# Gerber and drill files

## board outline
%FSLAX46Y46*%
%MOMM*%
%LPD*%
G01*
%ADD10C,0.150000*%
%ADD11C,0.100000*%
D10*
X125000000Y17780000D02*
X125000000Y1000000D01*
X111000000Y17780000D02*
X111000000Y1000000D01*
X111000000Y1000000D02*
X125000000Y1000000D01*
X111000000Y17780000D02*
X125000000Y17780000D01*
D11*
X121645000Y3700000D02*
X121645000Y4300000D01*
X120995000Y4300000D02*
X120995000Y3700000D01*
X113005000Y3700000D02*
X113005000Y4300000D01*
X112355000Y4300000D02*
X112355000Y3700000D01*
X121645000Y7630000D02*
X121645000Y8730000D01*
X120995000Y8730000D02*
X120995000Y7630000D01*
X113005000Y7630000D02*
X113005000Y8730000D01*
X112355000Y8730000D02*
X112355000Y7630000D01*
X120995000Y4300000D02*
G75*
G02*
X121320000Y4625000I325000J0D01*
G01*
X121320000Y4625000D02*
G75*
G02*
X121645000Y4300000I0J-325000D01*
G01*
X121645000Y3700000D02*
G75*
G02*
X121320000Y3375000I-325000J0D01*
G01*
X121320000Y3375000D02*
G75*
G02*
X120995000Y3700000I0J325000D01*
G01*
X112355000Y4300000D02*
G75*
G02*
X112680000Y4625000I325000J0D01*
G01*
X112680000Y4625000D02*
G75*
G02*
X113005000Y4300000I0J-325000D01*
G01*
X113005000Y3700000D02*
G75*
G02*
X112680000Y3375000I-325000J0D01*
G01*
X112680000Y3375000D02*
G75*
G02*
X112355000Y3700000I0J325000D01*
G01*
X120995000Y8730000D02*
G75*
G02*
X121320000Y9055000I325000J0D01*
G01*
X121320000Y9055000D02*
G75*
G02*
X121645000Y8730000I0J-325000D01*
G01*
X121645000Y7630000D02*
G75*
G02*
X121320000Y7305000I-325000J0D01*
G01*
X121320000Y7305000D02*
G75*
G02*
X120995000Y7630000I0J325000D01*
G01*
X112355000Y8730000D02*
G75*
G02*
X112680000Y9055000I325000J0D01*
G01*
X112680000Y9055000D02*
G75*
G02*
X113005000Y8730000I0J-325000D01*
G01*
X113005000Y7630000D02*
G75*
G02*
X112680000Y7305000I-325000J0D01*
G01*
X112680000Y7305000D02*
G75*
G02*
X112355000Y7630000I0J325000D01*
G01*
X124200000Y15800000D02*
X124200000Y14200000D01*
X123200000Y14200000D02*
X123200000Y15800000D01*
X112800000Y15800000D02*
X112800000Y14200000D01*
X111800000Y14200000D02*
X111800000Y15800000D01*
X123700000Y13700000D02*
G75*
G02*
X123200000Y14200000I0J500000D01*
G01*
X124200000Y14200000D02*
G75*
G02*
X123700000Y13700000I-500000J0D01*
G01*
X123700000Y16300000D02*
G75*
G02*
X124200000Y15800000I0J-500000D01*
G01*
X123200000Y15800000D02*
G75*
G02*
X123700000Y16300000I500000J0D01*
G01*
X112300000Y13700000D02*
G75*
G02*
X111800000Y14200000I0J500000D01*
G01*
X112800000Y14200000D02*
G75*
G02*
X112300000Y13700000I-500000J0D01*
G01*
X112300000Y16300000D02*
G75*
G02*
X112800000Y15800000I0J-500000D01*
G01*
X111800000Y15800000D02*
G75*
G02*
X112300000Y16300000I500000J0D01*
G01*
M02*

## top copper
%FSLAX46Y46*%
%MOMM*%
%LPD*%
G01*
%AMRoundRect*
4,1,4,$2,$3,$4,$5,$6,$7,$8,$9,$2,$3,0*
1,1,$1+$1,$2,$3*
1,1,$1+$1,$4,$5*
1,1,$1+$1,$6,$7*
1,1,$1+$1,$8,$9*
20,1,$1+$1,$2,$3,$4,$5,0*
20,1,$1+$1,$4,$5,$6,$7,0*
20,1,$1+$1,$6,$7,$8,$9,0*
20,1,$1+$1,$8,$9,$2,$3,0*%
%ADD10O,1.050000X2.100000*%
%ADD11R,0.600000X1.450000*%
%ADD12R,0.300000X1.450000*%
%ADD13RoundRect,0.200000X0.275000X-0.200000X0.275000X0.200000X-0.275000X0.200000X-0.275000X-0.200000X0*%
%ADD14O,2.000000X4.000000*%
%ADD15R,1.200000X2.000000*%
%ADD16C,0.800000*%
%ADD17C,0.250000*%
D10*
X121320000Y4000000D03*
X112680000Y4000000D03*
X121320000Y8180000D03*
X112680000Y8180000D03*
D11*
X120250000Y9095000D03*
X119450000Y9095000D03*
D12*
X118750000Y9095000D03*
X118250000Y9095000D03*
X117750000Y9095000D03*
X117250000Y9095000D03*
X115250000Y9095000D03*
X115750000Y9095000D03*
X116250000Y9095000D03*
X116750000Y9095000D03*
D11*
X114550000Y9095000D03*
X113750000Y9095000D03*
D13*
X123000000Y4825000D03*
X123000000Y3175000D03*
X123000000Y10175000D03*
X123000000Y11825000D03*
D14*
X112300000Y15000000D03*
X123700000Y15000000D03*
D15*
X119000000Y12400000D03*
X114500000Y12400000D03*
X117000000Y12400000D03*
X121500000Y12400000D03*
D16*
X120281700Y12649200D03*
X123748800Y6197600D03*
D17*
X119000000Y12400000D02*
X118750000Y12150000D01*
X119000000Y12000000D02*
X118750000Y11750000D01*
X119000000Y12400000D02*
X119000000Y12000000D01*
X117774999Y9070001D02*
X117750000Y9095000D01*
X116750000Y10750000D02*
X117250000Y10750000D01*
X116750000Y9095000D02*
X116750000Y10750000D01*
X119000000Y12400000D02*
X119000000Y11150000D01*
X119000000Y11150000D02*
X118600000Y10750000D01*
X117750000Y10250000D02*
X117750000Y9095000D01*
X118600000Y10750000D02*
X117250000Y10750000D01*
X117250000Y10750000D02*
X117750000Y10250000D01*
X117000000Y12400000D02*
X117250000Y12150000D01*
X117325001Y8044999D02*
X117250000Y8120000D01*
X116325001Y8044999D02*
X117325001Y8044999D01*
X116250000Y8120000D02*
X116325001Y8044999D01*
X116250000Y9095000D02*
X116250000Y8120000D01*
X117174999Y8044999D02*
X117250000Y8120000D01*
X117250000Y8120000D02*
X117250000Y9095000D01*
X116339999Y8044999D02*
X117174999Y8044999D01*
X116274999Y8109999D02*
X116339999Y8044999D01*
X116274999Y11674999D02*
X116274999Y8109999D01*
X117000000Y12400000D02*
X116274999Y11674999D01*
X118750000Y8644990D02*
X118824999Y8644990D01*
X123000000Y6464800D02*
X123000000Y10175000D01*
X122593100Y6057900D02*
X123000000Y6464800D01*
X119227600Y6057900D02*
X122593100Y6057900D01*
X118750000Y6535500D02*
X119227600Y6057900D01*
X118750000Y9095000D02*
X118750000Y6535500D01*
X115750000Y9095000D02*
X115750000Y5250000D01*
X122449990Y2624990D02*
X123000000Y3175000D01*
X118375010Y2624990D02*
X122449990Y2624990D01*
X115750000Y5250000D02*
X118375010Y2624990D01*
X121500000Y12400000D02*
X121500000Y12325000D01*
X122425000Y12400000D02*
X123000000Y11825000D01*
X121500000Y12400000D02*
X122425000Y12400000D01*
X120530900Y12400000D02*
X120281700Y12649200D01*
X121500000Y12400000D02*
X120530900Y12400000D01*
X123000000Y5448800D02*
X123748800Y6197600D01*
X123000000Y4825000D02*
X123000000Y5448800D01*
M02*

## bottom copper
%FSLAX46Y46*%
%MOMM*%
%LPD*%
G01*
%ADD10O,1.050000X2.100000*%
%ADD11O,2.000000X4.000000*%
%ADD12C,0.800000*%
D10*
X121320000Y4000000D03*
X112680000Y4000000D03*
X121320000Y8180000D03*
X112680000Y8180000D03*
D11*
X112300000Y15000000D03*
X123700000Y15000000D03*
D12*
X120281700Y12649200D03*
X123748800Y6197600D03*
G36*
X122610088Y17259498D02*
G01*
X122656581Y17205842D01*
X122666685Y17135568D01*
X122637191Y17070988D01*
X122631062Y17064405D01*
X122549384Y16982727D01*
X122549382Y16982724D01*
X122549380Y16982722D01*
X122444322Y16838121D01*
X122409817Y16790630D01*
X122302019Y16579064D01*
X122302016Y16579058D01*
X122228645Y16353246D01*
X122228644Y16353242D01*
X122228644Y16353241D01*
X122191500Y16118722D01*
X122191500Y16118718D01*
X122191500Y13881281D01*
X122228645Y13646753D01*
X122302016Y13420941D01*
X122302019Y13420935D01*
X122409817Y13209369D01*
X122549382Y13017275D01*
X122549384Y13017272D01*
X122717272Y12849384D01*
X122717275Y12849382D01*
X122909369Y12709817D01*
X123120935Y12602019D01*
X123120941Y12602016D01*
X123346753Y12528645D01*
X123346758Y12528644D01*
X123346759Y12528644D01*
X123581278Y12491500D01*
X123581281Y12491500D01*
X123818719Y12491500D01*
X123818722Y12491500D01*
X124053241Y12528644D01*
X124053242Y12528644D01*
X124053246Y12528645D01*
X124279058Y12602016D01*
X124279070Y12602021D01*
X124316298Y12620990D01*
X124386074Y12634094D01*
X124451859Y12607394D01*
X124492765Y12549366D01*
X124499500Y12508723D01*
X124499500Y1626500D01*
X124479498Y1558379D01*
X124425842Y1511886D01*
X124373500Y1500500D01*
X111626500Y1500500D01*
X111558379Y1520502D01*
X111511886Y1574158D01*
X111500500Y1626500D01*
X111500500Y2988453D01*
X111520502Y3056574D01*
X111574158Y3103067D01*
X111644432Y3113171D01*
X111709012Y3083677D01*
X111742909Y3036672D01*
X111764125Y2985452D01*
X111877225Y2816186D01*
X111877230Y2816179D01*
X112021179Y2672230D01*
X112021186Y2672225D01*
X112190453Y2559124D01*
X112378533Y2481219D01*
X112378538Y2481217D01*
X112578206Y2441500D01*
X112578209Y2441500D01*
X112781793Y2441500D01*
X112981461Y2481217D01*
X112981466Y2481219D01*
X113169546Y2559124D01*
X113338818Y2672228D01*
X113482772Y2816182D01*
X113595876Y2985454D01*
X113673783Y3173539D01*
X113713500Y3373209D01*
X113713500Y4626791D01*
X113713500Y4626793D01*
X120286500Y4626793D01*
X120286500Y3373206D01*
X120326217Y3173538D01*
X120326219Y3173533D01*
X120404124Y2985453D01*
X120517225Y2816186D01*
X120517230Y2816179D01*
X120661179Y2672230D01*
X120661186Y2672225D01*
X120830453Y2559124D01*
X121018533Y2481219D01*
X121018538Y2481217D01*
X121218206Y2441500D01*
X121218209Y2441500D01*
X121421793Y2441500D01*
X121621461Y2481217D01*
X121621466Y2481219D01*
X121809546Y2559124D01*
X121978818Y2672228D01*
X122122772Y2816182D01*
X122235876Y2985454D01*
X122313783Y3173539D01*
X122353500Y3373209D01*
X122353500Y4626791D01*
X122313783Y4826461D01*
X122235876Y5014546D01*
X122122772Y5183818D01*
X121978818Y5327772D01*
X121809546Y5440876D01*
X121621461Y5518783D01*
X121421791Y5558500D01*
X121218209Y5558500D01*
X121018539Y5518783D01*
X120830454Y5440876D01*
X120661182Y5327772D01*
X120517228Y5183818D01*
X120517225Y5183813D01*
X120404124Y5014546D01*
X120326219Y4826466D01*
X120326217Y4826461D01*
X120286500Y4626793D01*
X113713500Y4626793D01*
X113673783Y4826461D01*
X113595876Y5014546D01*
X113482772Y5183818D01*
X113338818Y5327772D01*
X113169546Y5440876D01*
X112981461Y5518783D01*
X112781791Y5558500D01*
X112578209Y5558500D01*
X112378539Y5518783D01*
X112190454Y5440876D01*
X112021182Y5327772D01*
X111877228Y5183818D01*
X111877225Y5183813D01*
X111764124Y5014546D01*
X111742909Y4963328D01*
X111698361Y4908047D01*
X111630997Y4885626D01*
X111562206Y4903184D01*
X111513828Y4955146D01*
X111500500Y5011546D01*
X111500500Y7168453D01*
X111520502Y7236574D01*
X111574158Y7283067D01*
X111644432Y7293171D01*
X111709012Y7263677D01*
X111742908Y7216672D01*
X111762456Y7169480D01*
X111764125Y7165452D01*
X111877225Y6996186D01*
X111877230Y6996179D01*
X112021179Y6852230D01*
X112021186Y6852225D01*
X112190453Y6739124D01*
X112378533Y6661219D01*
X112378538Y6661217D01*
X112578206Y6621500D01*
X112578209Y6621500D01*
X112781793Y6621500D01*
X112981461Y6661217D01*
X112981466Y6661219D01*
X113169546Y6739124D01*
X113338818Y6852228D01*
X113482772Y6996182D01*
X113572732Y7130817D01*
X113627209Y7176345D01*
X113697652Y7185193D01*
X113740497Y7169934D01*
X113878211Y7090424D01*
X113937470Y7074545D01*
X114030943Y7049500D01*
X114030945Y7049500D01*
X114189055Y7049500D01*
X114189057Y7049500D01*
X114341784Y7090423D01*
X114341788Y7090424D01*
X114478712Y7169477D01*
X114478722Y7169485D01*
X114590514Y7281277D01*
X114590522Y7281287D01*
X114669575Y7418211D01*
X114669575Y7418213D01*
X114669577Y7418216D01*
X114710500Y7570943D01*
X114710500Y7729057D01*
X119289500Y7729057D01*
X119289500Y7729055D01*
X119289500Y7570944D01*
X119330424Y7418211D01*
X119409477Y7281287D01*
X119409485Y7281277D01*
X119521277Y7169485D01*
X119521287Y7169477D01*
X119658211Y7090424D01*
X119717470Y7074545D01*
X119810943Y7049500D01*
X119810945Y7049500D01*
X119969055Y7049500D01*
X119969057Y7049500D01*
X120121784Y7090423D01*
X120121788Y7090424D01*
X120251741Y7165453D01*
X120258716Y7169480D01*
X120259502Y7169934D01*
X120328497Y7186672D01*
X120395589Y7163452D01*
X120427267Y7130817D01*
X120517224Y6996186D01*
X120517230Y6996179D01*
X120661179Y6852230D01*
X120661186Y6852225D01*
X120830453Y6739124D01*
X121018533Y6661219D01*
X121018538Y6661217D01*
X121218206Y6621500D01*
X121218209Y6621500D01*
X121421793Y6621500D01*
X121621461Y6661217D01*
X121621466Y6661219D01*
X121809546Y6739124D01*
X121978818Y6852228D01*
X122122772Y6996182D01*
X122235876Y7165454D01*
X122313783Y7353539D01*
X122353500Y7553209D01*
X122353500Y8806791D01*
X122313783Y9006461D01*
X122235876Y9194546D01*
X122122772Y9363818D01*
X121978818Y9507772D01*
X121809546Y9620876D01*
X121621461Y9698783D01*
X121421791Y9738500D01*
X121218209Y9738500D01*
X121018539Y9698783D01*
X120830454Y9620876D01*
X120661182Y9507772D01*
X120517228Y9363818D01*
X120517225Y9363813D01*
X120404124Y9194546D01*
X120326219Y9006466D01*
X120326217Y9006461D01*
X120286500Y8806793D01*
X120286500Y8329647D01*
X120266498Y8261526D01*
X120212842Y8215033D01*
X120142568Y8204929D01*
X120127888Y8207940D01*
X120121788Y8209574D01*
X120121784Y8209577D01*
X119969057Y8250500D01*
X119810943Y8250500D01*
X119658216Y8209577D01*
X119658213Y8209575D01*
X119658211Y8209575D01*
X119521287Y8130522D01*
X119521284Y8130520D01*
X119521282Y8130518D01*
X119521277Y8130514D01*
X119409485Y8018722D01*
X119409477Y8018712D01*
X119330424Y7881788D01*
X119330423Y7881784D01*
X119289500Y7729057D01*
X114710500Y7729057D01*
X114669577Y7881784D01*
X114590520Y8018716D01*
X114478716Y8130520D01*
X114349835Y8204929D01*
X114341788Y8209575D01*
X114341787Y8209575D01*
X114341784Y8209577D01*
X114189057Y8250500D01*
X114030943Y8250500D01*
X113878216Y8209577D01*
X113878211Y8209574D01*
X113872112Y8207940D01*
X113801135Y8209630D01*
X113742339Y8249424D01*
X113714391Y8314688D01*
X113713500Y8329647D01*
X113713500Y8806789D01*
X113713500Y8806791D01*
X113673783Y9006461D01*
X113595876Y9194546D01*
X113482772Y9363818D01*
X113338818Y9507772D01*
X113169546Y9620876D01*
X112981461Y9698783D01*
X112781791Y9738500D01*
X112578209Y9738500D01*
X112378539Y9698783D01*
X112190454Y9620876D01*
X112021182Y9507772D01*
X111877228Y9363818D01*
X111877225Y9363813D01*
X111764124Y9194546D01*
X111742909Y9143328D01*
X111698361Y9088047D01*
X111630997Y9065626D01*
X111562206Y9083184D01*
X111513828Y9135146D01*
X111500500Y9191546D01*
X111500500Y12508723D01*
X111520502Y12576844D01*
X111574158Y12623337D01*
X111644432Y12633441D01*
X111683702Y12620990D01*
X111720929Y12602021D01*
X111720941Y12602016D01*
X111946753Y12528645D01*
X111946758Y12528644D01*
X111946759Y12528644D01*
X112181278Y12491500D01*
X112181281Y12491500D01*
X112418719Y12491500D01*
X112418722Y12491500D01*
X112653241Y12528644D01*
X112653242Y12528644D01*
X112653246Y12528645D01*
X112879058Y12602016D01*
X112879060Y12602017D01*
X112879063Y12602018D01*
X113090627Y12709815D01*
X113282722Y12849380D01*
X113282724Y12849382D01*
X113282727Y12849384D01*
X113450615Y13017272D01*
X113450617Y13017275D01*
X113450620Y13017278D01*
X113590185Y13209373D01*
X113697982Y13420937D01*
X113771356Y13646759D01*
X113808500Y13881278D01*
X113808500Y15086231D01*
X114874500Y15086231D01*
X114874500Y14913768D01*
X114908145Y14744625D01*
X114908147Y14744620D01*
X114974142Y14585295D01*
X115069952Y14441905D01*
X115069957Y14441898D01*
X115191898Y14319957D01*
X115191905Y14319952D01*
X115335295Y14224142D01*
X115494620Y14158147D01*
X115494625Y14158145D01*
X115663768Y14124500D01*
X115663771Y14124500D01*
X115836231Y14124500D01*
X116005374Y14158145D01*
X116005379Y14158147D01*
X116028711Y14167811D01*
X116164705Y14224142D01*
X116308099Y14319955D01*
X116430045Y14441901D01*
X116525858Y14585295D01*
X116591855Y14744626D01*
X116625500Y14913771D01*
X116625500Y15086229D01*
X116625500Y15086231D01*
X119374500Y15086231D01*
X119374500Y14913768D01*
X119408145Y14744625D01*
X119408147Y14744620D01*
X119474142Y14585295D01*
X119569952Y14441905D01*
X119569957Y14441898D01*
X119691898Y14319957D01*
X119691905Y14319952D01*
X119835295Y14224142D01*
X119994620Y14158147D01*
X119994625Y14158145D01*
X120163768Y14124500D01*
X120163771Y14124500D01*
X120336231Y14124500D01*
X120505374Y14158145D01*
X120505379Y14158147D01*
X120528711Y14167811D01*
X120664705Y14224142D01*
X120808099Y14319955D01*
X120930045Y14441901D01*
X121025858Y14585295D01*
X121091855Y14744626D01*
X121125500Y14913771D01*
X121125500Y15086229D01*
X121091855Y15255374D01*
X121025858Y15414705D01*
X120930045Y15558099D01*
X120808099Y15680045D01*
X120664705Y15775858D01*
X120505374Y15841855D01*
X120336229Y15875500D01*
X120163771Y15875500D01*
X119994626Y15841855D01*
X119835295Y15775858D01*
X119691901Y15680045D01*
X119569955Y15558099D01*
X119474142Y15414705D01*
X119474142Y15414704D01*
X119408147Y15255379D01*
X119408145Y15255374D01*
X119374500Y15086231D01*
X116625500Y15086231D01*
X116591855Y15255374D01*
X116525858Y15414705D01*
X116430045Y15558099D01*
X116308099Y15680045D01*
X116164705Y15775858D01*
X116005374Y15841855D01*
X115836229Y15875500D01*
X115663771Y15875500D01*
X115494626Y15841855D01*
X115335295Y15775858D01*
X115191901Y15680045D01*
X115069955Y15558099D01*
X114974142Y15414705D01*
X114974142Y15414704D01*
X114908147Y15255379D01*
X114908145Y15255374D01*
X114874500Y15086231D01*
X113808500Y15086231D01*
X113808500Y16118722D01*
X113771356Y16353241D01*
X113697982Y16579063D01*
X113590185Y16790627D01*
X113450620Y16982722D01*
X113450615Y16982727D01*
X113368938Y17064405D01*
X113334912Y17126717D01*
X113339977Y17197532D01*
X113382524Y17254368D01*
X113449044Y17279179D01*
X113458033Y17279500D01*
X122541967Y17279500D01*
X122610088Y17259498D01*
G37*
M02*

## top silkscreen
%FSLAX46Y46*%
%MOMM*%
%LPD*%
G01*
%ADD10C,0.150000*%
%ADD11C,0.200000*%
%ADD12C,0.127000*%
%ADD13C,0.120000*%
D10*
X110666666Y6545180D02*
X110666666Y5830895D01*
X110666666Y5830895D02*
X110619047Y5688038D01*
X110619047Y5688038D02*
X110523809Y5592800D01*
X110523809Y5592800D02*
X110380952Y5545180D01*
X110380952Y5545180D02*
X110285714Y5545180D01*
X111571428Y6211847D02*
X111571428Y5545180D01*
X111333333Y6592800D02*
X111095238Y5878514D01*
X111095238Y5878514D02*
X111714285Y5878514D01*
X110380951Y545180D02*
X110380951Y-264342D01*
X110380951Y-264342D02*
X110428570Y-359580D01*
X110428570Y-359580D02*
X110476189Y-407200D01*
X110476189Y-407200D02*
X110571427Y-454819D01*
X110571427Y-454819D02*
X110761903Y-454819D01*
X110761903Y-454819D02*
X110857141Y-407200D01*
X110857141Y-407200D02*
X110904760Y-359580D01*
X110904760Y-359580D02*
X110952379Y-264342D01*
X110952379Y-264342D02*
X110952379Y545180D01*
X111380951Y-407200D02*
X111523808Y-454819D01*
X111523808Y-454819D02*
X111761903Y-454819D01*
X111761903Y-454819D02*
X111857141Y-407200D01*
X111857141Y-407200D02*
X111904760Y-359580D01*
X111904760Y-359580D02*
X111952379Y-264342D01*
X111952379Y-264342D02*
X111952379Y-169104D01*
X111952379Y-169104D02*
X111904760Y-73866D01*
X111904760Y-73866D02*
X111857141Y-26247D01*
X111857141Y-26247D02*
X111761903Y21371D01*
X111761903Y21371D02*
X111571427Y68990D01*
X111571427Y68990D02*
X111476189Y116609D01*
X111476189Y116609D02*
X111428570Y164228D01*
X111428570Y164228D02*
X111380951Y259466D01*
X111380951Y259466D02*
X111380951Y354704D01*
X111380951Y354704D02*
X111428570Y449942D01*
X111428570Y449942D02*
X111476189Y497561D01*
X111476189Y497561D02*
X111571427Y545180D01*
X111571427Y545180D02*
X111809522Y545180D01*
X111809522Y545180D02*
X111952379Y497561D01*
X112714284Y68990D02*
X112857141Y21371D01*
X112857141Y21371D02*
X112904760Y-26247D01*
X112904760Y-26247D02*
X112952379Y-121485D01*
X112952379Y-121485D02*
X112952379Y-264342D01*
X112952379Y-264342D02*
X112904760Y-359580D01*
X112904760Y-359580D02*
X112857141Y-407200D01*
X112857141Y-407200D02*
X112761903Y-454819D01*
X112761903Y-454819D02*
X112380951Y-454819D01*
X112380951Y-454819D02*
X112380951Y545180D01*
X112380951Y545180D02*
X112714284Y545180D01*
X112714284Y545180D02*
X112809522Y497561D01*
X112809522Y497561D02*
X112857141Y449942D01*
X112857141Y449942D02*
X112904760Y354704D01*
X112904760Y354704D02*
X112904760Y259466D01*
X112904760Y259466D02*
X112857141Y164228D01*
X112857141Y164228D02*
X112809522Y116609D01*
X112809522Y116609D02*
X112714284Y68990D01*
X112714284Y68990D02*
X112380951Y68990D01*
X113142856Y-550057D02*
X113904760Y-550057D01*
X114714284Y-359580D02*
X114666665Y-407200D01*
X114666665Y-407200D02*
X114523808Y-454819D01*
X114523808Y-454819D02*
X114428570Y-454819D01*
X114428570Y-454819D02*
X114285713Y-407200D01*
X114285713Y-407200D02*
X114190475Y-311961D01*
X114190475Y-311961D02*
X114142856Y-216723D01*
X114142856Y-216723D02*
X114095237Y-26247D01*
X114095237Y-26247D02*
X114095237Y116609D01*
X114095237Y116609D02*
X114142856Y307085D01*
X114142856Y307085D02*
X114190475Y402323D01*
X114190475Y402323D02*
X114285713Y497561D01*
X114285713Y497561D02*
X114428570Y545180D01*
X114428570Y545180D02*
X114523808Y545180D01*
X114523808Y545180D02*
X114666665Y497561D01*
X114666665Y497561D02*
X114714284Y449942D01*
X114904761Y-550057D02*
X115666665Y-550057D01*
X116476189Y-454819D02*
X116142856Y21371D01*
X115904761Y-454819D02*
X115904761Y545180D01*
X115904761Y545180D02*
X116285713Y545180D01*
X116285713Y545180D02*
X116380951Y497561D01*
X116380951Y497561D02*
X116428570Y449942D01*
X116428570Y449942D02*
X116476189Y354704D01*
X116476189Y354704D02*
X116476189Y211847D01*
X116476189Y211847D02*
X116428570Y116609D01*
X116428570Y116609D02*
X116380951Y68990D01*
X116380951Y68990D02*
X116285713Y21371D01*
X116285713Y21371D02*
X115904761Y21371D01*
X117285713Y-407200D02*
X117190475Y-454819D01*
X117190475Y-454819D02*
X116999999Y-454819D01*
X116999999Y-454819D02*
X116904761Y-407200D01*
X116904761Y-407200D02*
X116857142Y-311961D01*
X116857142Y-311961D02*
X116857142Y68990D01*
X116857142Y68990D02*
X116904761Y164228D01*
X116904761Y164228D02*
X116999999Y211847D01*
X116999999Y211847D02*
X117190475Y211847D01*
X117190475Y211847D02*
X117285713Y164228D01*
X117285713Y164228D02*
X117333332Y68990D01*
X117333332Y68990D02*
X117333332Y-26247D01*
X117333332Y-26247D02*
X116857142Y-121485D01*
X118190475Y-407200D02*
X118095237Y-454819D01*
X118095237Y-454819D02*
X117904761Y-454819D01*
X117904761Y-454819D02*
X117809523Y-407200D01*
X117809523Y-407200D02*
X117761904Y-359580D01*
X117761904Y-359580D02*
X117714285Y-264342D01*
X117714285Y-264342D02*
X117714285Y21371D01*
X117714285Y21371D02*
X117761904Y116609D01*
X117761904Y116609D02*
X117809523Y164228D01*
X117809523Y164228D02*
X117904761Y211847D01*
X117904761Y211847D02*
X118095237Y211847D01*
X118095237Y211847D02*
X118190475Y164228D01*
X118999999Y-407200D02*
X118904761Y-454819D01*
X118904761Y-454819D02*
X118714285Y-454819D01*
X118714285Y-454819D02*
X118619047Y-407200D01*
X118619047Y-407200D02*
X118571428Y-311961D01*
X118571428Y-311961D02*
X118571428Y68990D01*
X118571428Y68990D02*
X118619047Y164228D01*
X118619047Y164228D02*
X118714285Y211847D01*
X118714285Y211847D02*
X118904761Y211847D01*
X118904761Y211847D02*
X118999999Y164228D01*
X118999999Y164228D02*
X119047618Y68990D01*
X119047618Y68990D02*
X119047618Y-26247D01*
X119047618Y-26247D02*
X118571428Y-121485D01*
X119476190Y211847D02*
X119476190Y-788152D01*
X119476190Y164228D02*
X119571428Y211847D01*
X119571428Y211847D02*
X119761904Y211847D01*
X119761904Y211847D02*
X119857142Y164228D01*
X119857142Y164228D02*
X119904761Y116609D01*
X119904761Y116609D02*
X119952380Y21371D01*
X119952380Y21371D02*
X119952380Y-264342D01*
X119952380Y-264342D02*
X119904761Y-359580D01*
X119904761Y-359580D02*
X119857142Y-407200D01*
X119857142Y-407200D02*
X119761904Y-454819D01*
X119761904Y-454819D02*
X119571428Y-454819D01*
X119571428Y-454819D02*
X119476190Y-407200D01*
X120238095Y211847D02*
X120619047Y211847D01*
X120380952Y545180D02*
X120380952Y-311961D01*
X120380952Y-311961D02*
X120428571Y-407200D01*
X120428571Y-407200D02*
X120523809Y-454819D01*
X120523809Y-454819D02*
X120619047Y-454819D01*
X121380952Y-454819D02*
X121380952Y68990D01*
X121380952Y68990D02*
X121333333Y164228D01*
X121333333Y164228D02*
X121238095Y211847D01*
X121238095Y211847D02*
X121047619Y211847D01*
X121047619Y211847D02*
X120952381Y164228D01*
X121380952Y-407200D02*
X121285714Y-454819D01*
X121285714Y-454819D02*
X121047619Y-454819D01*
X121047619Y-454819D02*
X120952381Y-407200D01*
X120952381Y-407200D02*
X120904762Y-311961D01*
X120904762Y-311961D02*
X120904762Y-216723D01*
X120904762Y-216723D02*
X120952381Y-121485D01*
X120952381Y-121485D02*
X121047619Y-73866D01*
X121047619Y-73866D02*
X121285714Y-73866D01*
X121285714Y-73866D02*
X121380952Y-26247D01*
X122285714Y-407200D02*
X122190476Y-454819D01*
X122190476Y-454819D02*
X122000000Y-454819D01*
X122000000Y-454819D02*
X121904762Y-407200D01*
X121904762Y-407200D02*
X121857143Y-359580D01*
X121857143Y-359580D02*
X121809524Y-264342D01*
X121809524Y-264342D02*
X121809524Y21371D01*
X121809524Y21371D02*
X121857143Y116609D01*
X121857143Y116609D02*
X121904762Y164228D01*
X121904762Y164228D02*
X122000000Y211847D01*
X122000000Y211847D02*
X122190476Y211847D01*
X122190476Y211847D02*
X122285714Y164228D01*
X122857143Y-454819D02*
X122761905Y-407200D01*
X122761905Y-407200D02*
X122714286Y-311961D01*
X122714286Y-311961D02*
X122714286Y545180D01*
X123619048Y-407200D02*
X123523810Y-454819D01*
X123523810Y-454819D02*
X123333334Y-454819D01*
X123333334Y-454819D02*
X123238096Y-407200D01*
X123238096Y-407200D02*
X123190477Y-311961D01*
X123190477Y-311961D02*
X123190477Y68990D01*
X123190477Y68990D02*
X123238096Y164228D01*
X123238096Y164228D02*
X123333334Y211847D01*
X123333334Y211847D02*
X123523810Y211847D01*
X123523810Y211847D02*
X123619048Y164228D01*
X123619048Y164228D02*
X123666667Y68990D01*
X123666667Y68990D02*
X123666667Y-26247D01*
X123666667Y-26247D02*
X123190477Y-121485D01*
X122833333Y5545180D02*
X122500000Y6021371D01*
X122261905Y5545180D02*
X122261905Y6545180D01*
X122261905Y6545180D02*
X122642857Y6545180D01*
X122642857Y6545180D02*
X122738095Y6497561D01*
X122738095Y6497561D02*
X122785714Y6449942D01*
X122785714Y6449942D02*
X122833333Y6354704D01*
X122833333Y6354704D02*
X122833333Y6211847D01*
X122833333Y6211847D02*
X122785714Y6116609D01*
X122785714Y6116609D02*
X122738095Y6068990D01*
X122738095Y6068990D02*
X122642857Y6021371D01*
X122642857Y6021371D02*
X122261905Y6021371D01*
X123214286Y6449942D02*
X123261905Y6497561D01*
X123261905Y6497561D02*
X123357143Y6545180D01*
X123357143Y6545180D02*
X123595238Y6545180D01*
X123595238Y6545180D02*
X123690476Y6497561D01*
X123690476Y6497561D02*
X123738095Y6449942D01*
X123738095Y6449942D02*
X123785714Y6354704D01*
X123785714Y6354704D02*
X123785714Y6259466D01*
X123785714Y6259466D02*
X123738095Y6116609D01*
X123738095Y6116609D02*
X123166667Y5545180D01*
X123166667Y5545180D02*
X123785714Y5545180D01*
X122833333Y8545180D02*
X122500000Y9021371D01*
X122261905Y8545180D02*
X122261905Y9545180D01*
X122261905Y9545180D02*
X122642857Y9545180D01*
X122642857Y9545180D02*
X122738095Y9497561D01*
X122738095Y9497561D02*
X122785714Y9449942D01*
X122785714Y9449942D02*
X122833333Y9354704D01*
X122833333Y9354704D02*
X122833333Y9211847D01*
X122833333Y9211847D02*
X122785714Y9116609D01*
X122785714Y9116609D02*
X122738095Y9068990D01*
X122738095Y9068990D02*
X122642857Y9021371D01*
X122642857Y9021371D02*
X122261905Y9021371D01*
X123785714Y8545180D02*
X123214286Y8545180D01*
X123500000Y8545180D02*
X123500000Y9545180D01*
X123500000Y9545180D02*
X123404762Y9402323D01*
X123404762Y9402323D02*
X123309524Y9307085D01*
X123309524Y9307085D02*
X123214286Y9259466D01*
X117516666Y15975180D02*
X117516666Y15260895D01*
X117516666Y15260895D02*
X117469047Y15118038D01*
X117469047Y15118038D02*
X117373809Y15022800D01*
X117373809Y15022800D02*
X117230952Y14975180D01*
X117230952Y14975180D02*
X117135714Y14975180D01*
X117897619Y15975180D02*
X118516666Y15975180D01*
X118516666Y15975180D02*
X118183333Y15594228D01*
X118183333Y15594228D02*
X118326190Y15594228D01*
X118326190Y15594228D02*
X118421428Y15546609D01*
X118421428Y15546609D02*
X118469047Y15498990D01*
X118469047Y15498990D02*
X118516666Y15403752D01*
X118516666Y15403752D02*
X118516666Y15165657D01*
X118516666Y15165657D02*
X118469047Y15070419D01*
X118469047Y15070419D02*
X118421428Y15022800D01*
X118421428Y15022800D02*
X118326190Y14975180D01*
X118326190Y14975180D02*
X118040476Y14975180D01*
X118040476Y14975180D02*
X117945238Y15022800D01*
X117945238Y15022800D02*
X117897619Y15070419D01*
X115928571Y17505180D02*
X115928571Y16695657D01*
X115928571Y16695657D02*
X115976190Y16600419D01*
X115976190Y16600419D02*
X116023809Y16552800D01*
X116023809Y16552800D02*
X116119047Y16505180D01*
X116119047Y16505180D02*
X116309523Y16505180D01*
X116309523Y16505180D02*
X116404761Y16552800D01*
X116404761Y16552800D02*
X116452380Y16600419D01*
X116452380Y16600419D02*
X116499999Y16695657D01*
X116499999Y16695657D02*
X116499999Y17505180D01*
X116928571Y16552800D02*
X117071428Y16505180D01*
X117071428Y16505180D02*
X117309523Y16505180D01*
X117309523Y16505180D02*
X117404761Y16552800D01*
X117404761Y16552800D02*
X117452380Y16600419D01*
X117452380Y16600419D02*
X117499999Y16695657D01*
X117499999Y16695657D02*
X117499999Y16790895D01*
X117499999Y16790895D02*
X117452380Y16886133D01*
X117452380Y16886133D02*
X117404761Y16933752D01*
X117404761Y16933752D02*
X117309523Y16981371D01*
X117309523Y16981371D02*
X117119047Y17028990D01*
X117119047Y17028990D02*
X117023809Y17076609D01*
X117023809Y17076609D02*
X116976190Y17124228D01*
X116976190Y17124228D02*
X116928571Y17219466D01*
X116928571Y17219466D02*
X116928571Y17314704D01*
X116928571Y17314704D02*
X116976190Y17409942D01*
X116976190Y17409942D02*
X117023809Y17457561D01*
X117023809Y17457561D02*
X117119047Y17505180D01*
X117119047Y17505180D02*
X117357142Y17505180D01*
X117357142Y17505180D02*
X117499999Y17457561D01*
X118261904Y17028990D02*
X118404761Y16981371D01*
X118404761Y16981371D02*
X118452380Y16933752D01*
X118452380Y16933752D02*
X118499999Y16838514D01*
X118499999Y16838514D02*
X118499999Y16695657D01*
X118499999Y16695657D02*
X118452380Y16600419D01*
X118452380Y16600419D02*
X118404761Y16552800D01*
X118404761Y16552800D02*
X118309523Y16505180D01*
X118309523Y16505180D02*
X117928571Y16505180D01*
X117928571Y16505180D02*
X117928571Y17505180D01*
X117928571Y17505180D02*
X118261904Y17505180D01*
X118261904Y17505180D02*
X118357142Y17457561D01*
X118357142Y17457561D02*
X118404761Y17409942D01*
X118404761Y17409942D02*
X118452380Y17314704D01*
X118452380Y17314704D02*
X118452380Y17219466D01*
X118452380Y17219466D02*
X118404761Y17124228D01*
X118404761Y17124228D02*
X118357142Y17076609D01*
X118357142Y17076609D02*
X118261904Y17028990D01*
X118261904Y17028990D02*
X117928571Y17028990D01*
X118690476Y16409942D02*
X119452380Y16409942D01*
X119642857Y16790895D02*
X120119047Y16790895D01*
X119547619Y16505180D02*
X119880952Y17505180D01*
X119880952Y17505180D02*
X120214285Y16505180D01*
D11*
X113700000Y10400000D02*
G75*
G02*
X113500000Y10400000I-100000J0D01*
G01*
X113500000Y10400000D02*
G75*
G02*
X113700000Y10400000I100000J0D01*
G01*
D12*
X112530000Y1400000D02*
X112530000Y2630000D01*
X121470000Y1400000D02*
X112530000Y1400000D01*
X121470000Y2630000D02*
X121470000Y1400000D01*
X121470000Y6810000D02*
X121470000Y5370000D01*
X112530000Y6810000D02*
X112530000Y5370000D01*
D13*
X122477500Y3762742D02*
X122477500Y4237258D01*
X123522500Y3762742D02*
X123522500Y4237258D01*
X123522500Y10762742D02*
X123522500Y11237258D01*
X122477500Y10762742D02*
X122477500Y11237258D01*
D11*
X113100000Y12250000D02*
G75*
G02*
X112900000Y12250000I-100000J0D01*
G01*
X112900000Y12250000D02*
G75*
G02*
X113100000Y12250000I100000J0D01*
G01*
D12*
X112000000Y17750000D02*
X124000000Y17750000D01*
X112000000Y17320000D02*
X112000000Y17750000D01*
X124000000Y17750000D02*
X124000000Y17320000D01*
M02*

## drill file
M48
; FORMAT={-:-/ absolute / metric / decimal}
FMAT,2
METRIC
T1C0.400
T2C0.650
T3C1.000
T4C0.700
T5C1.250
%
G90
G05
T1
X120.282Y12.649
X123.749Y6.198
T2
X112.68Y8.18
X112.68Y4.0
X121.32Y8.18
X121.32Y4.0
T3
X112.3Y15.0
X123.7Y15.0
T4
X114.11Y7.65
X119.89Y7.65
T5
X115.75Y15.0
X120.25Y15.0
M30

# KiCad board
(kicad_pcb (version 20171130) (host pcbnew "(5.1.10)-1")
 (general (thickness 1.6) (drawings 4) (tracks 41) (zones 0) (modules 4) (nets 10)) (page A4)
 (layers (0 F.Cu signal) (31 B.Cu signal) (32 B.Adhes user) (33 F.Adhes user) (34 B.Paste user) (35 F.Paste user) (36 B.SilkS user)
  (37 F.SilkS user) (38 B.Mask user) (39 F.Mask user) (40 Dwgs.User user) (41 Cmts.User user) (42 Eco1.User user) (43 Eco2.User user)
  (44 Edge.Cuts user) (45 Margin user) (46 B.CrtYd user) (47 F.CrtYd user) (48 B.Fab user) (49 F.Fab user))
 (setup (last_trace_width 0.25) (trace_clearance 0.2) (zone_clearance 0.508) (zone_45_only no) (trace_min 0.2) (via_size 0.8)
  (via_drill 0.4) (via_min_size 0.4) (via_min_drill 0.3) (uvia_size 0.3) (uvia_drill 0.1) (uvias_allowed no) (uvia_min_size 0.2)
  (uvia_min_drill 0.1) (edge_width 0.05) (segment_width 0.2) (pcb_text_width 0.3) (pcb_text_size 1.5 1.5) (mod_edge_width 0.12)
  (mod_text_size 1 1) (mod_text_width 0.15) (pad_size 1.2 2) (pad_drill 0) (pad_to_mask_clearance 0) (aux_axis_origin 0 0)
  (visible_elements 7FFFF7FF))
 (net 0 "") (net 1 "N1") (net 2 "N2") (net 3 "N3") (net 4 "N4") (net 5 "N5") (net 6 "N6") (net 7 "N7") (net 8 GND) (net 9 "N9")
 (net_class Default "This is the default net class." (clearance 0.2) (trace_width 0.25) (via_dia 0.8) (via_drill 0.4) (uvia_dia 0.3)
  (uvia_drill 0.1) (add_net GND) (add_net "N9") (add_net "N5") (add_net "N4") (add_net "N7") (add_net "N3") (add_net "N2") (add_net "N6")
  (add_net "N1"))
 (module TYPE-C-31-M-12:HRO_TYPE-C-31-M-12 (layer F.Cu) (at 117 -4)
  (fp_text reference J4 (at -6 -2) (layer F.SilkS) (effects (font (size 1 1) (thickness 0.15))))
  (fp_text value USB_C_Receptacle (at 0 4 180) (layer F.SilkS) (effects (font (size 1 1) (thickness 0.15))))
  (fp_circle (center -3.4 -6.4) (end -3.3 -6.4) (layer F.SilkS) (width 0.2))
  (fp_line (start -4.47 2.6) (end -4.47 1.37) (layer F.SilkS) (width 0.127))
  (fp_line (start 4.47 2.6) (end -4.47 2.6) (layer F.SilkS) (width 0.127))
  (fp_line (start 4.47 1.37) (end 4.47 2.6) (layer F.SilkS) (width 0.127))
  (fp_line (start 4.47 -2.81) (end 4.47 -1.37) (layer F.SilkS) (width 0.127))
  (fp_line (start -4.47 -2.81) (end -4.47 -1.37) (layer F.SilkS) (width 0.127))
  (fp_line (start 4.645 0.3) (end 4.645 -0.3) (layer Edge.Cuts) (width 0.1))
  (fp_line (start 3.995 -0.3) (end 3.995 0.3) (layer Edge.Cuts) (width 0.1))
  (fp_line (start -3.995 0.3) (end -3.995 -0.3) (layer Edge.Cuts) (width 0.1))
  (fp_line (start -4.645 -0.3) (end -4.645 0.3) (layer Edge.Cuts) (width 0.1))
  (fp_line (start 4.645 -3.63) (end 4.645 -4.73) (layer Edge.Cuts) (width 0.1))
  (fp_line (start 3.995 -4.73) (end 3.995 -3.63) (layer Edge.Cuts) (width 0.1))
  (fp_line (start -3.995 -3.63) (end -3.995 -4.73) (layer Edge.Cuts) (width 0.1))
  (fp_line (start -4.645 -4.73) (end -4.645 -3.63) (layer Edge.Cuts) (width 0.1))
  (fp_arc (start 4.32 -0.3) (end 3.995 -0.3) (angle 90) (layer Edge.Cuts) (width 0.1))
  (fp_arc (start 4.32 -0.3) (end 4.32 -0.625) (angle 90) (layer Edge.Cuts) (width 0.1))
  (fp_arc (start 4.32 0.3) (end 4.645 0.3) (angle 90) (layer Edge.Cuts) (width 0.1))
  (fp_arc (start 4.32 0.3) (end 4.32 0.625) (angle 90) (layer Edge.Cuts) (width 0.1))
  (fp_arc (start -4.32 -0.3) (end -4.645 -0.3) (angle 90) (layer Edge.Cuts) (width 0.1))
  (fp_arc (start -4.32 -0.3) (end -4.32 -0.625) (angle 90) (layer Edge.Cuts) (width 0.1))
  (fp_arc (start -4.32 0.3) (end -3.995 0.3) (angle 90) (layer Edge.Cuts) (width 0.1))
  (fp_arc (start -4.32 0.3) (end -4.32 0.625) (angle 90) (layer Edge.Cuts) (width 0.1))
  (fp_arc (start 4.32 -4.73) (end 3.995 -4.73) (angle 90) (layer Edge.Cuts) (width 0.1))
  (fp_arc (start 4.32 -4.73) (end 4.32 -5.055) (angle 90) (layer Edge.Cuts) (width 0.1))
  (fp_arc (start 4.32 -3.63) (end 4.645 -3.63) (angle 90) (layer Edge.Cuts) (width 0.1))
  (fp_arc (start 4.32 -3.63) (end 4.32 -3.305) (angle 90) (layer Edge.Cuts) (width 0.1))
  (fp_arc (start -4.32 -4.73) (end -4.645 -4.73) (angle 90) (layer Edge.Cuts) (width 0.1))
  (fp_arc (start -4.32 -4.73) (end -4.32 -5.055) (angle 90) (layer Edge.Cuts) (width 0.1))
  (fp_arc (start -4.32 -3.63) (end -3.995 -3.63) (angle 90) (layer Edge.Cuts) (width 0.1))
  (fp_arc (start -4.32 -3.63) (end -4.32 -3.305) (angle 90) (layer Edge.Cuts) (width 0.1))
  (pad Hole np_thru_hole circle (at 2.89 -3.65) (size 0.7 0.7) (drill 0.7) (layers *.Cu *.Mask))
  (pad Hole np_thru_hole circle (at -2.89 -3.65) (size 0.7 0.7) (drill 0.7) (layers *.Cu *.Mask))
  (pad S4 thru_hole oval (at 4.32 0 90) (size 2.1 1.05) (drill 0.65) (layers *.Cu *.Mask))
  (pad S3 thru_hole oval (at -4.32 0 90) (size 2.1 1.05) (drill 0.65) (layers *.Cu *.Mask))
  (pad S2 thru_hole oval (at 4.32 -4.18 90) (size 2.1 1.05) (drill 0.65) (layers *.Cu *.Mask))
  (pad S1 thru_hole oval (at -4.32 -4.18 90) (size 2.1 1.05) (drill 0.65) (layers *.Cu *.Mask) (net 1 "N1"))
  (pad B1A12 smd rect (at 3.25 -5.095) (size 0.6 1.45) (layers F.Cu F.Paste))
  (pad B4A9 smd rect (at 2.45 -5.095) (size 0.6 1.45) (layers F.Cu F.Paste))
  (pad B5 smd rect (at 1.75 -5.095) (size 0.3 1.45) (layers F.Cu F.Paste) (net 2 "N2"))
  (pad A8 smd rect (at 1.25 -5.095) (size 0.3 1.45) (layers F.Cu F.Paste) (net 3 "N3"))
  (pad B6 smd rect (at 0.75 -5.095) (size 0.3 1.45) (layers F.Cu F.Paste) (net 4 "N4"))
  (pad A7 smd rect (at 0.25 -5.095) (size 0.3 1.45) (layers F.Cu F.Paste) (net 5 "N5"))
  (pad B8 smd rect (at -1.75 -5.095) (size 0.3 1.45) (layers F.Cu F.Paste) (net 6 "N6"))
  (pad A5 smd rect (at -1.25 -5.095) (size 0.3 1.45) (layers F.Cu F.Paste) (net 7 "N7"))
  (pad B7 smd rect (at -0.75 -5.095) (size 0.3 1.45) (layers F.Cu F.Paste) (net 5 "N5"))
  (pad A6 smd rect (at -0.25 -5.095) (size 0.3 1.45) (layers F.Cu F.Paste) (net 4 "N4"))
  (pad A4B9 smd rect (at -2.45 -5.095) (size 0.6 1.45) (layers F.Cu F.Paste))
  (pad A1B12 smd rect (at -3.25 -5.095) (size 0.6 1.45) (layers F.Cu F.Paste)))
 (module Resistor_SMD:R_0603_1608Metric (layer F.Cu) (at 123 -4 90)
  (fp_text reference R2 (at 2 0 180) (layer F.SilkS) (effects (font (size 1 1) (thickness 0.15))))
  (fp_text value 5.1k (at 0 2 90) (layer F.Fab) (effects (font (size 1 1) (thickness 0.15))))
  (fp_line (start -0.237258 -0.5225) (end 0.237258 -0.5225) (layer F.SilkS) (width 0.12))
  (fp_line (start -0.237258 0.5225) (end 0.237258 0.5225) (layer F.SilkS) (width 0.12))
  (pad 2 smd roundrect (at 0.825 0 90) (size 0.8 0.95) (layers F.Cu F.Paste F.Mask) (roundrect_rratio 0.25) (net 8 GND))
  (pad 1 smd roundrect (at -0.825 0 90) (size 0.8 0.95) (layers F.Cu F.Paste F.Mask) (roundrect_rratio 0.25) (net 7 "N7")))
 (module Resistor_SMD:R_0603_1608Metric (layer F.Cu) (at 123 -11 90)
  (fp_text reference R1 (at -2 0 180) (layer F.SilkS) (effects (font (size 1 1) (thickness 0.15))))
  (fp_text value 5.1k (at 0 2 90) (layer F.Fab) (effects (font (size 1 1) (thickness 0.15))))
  (fp_line (start -0.237258 0.5225) (end 0.237258 0.5225) (layer F.SilkS) (width 0.12))
  (fp_line (start -0.237258 -0.5225) (end 0.237258 -0.5225) (layer F.SilkS) (width 0.12))
  (pad 1 smd roundrect (at -0.825 0 90) (size 0.8 0.95) (layers F.Cu F.Paste F.Mask) (roundrect_rratio 0.25) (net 2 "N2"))
  (pad 2 smd roundrect (at 0.825 0 90) (size 0.8 0.95) (layers F.Cu F.Paste F.Mask) (roundrect_rratio 0.25) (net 8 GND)))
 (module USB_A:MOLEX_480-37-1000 (layer F.Cu) (at 118 -15 180)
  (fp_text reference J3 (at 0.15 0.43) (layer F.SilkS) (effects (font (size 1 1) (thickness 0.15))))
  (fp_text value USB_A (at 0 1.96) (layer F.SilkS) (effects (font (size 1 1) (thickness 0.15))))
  (fp_line (start -6.2 0.8) (end -6.2 -0.8) (layer Edge.Cuts) (width 0.1))
  (fp_line (start -5.2 -0.8) (end -5.2 0.8) (layer Edge.Cuts) (width 0.1))
  (fp_line (start 5.2 0.8) (end 5.2 -0.8) (layer Edge.Cuts) (width 0.1))
  (fp_line (start 6.2 -0.8) (end 6.2 0.8) (layer Edge.Cuts) (width 0.1))
  (fp_circle (center 5 -2.75) (end 5.1 -2.75) (layer F.SilkS) (width 0.2))
  (fp_line (start 6 2.75) (end -6 2.75) (layer F.SilkS) (width 0.127))
  (fp_line (start 6 2.32) (end 6 2.75) (layer F.SilkS) (width 0.127))
  (fp_line (start -6 2.75) (end -6 2.32) (layer F.SilkS) (width 0.127))
  (fp_arc (start -5.7 -0.8) (end -5.2 -0.8) (angle -90) (layer Edge.Cuts) (width 0.1))
  (fp_arc (start -5.7 -0.8) (end -5.7 -1.3) (angle -90) (layer Edge.Cuts) (width 0.1))
  (fp_arc (start -5.7 0.8) (end -6.2 0.8) (angle -90) (layer Edge.Cuts) (width 0.1))
  (fp_arc (start -5.7 0.8) (end -5.7 1.3) (angle -90) (layer Edge.Cuts) (width 0.1))
  (fp_arc (start 5.7 -0.8) (end 6.2 -0.8) (angle -90) (layer Edge.Cuts) (width 0.1))
  (fp_arc (start 5.7 -0.8) (end 5.7 -1.3) (angle -90) (layer Edge.Cuts) (width 0.1))
  (fp_arc (start 5.7 0.8) (end 5.2 0.8) (angle -90) (layer Edge.Cuts) (width 0.1))
  (fp_arc (start 5.7 0.8) (end 5.7 1.3) (angle -90) (layer Edge.Cuts) (width 0.1))
  (pad S2 thru_hole oval (at 5.7 0 270) (size 4 2) (drill 1) (layers *.Cu *.Mask))
  (pad S1 thru_hole oval (at -5.7 0 270) (size 4 2) (drill 1) (layers *.Cu *.Mask))
  (pad 3 smd rect (at -1 -2.6 180) (size 1.2 2) (layers F.Cu F.Paste) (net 4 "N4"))
  (pad 1 smd rect (at 3.5 -2.6 180) (size 1.2 2) (layers F.Cu F.Paste) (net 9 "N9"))
  (pad 2 smd rect (at 1 -2.6 180) (size 1.2 2) (layers F.Cu F.Paste) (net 5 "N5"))
  (pad 4 smd rect (at -3.5 -2.6 180) (size 1.2 2) (layers F.Cu F.Paste) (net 8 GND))
  (pad Hole np_thru_hole circle (at 2.25 0 180) (size 1.25 1.25) (drill 1.25) (layers *.Cu *.Mask))
  (pad Hole np_thru_hole circle (at -2.25 0 180) (size 1.25 1.25) (drill 1.25) (layers *.Cu *.Mask)))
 (gr_line (start 125 -17.78) (end 125 -1) (layer Edge.Cuts) (width 0.15))
 (gr_line (start 111 -17.78) (end 111 -1) (layer Edge.Cuts) (width 0.15))
 (gr_line (start 111 -1) (end 125 -1) (layer Edge.Cuts) (width 0.15))
 (gr_line (start 111 -17.78) (end 125 -17.78) (layer Edge.Cuts) (width 0.15))
 (segment (start 119 -12.4) (end 118.75 -12.15) (width 0.25) (layer F.Cu) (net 4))
 (segment (start 119 -12) (end 118.75 -11.75) (width 0.25) (layer F.Cu) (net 4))
 (segment (start 119 -12.4) (end 119 -12) (width 0.25) (layer F.Cu) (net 4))
 (segment (start 117.774999 -9.070001) (end 117.75 -9.095) (width 0.25) (layer F.Cu) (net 4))
 (segment (start 116.75 -10.75) (end 117.25 -10.75) (width 0.25) (layer F.Cu) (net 4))
 (segment (start 116.75 -9.095) (end 116.75 -10.75) (width 0.25) (layer F.Cu) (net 4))
 (segment (start 119 -12.4) (end 119 -11.15) (width 0.25) (layer F.Cu) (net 4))
 (segment (start 119 -11.15) (end 118.6 -10.75) (width 0.25) (layer F.Cu) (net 4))
 (segment (start 117.75 -10.25) (end 117.75 -9.095) (width 0.25) (layer F.Cu) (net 4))
 (segment (start 118.6 -10.75) (end 117.25 -10.75) (width 0.25) (layer F.Cu) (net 4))
 (segment (start 117.25 -10.75) (end 117.75 -10.25) (width 0.25) (layer F.Cu) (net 4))
 (segment (start 117 -12.4) (end 117.25 -12.15) (width 0.25) (layer F.Cu) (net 5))
 (segment (start 117.325001 -8.044999) (end 117.25 -8.12) (width 0.25) (layer F.Cu) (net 5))
 (segment (start 116.325001 -8.044999) (end 117.325001 -8.044999) (width 0.25) (layer F.Cu) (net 5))
 (segment (start 116.25 -8.12) (end 116.325001 -8.044999) (width 0.25) (layer F.Cu) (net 5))
 (segment (start 116.25 -9.095) (end 116.25 -8.12) (width 0.25) (layer F.Cu) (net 5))
 (segment (start 117.174999 -8.044999) (end 117.25 -8.12) (width 0.25) (layer F.Cu) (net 5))
 (segment (start 117.25 -8.12) (end 117.25 -9.095) (width 0.25) (layer F.Cu) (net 5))
 (segment (start 116.339999 -8.044999) (end 117.174999 -8.044999) (width 0.25) (layer F.Cu) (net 5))
 (segment (start 116.274999 -8.109999) (end 116.339999 -8.044999) (width 0.25) (layer F.Cu) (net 5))
 (segment (start 116.274999 -11.674999) (end 116.274999 -8.109999) (width 0.25) (layer F.Cu) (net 5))
 (segment (start 117 -12.4) (end 116.274999 -11.674999) (width 0.25) (layer F.Cu) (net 5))
 (segment (start 118.75 -8.64499) (end 118.824999 -8.64499) (width 0.25) (layer F.Cu) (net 2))
 (segment (start 123 -6.4648) (end 123 -10.175) (width 0.25) (layer F.Cu) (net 2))
 (segment (start 122.5931 -6.0579) (end 123 -6.4648) (width 0.25) (layer F.Cu) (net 2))
 (segment (start 119.2276 -6.0579) (end 122.5931 -6.0579) (width 0.25) (layer F.Cu) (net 2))
 (segment (start 118.75 -6.5355) (end 119.2276 -6.0579) (width 0.25) (layer F.Cu) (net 2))
 (segment (start 118.75 -9.095) (end 118.75 -6.5355) (width 0.25) (layer F.Cu) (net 2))
 (segment (start 115.75 -9.095) (end 115.75 -5.25) (width 0.25) (layer F.Cu) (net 7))
 (segment (start 122.44999 -2.62499) (end 123 -3.175) (width 0.25) (layer F.Cu) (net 7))
 (segment (start 118.37501 -2.62499) (end 122.44999 -2.62499) (width 0.25) (layer F.Cu) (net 7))
 (segment (start 115.75 -5.25) (end 118.37501 -2.62499) (width 0.25) (layer F.Cu) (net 7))
 (segment (start 121.5 -12.4) (end 121.5 -12.325) (width 0.25) (layer F.Cu) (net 8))
 (segment (start 122.425 -12.4) (end 123 -11.825) (width 0.25) (layer F.Cu) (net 8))
 (segment (start 121.5 -12.4) (end 122.425 -12.4) (width 0.25) (layer F.Cu) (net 8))
 (via (at 120.2817 -12.6492) (size 0.8) (drill 0.4) (layers F.Cu B.Cu) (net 8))
 (segment (start 120.5309 -12.4) (end 120.2817 -12.6492) (width 0.25) (layer F.Cu) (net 8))
 (segment (start 121.5 -12.4) (end 120.5309 -12.4) (width 0.25) (layer F.Cu) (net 8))
 (via (at 123.7488 -6.1976) (size 0.8) (drill 0.4) (layers F.Cu B.Cu) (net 8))
 (segment (start 123 -5.4488) (end 123.7488 -6.1976) (width 0.25) (layer F.Cu) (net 8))
 (segment (start 123 -4.825) (end 123 -5.4488) (width 0.25) (layer F.Cu) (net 8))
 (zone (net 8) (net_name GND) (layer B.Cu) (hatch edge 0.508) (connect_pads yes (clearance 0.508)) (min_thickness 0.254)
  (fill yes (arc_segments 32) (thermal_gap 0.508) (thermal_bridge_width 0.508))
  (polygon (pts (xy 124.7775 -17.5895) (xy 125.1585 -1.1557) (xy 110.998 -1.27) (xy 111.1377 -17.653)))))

